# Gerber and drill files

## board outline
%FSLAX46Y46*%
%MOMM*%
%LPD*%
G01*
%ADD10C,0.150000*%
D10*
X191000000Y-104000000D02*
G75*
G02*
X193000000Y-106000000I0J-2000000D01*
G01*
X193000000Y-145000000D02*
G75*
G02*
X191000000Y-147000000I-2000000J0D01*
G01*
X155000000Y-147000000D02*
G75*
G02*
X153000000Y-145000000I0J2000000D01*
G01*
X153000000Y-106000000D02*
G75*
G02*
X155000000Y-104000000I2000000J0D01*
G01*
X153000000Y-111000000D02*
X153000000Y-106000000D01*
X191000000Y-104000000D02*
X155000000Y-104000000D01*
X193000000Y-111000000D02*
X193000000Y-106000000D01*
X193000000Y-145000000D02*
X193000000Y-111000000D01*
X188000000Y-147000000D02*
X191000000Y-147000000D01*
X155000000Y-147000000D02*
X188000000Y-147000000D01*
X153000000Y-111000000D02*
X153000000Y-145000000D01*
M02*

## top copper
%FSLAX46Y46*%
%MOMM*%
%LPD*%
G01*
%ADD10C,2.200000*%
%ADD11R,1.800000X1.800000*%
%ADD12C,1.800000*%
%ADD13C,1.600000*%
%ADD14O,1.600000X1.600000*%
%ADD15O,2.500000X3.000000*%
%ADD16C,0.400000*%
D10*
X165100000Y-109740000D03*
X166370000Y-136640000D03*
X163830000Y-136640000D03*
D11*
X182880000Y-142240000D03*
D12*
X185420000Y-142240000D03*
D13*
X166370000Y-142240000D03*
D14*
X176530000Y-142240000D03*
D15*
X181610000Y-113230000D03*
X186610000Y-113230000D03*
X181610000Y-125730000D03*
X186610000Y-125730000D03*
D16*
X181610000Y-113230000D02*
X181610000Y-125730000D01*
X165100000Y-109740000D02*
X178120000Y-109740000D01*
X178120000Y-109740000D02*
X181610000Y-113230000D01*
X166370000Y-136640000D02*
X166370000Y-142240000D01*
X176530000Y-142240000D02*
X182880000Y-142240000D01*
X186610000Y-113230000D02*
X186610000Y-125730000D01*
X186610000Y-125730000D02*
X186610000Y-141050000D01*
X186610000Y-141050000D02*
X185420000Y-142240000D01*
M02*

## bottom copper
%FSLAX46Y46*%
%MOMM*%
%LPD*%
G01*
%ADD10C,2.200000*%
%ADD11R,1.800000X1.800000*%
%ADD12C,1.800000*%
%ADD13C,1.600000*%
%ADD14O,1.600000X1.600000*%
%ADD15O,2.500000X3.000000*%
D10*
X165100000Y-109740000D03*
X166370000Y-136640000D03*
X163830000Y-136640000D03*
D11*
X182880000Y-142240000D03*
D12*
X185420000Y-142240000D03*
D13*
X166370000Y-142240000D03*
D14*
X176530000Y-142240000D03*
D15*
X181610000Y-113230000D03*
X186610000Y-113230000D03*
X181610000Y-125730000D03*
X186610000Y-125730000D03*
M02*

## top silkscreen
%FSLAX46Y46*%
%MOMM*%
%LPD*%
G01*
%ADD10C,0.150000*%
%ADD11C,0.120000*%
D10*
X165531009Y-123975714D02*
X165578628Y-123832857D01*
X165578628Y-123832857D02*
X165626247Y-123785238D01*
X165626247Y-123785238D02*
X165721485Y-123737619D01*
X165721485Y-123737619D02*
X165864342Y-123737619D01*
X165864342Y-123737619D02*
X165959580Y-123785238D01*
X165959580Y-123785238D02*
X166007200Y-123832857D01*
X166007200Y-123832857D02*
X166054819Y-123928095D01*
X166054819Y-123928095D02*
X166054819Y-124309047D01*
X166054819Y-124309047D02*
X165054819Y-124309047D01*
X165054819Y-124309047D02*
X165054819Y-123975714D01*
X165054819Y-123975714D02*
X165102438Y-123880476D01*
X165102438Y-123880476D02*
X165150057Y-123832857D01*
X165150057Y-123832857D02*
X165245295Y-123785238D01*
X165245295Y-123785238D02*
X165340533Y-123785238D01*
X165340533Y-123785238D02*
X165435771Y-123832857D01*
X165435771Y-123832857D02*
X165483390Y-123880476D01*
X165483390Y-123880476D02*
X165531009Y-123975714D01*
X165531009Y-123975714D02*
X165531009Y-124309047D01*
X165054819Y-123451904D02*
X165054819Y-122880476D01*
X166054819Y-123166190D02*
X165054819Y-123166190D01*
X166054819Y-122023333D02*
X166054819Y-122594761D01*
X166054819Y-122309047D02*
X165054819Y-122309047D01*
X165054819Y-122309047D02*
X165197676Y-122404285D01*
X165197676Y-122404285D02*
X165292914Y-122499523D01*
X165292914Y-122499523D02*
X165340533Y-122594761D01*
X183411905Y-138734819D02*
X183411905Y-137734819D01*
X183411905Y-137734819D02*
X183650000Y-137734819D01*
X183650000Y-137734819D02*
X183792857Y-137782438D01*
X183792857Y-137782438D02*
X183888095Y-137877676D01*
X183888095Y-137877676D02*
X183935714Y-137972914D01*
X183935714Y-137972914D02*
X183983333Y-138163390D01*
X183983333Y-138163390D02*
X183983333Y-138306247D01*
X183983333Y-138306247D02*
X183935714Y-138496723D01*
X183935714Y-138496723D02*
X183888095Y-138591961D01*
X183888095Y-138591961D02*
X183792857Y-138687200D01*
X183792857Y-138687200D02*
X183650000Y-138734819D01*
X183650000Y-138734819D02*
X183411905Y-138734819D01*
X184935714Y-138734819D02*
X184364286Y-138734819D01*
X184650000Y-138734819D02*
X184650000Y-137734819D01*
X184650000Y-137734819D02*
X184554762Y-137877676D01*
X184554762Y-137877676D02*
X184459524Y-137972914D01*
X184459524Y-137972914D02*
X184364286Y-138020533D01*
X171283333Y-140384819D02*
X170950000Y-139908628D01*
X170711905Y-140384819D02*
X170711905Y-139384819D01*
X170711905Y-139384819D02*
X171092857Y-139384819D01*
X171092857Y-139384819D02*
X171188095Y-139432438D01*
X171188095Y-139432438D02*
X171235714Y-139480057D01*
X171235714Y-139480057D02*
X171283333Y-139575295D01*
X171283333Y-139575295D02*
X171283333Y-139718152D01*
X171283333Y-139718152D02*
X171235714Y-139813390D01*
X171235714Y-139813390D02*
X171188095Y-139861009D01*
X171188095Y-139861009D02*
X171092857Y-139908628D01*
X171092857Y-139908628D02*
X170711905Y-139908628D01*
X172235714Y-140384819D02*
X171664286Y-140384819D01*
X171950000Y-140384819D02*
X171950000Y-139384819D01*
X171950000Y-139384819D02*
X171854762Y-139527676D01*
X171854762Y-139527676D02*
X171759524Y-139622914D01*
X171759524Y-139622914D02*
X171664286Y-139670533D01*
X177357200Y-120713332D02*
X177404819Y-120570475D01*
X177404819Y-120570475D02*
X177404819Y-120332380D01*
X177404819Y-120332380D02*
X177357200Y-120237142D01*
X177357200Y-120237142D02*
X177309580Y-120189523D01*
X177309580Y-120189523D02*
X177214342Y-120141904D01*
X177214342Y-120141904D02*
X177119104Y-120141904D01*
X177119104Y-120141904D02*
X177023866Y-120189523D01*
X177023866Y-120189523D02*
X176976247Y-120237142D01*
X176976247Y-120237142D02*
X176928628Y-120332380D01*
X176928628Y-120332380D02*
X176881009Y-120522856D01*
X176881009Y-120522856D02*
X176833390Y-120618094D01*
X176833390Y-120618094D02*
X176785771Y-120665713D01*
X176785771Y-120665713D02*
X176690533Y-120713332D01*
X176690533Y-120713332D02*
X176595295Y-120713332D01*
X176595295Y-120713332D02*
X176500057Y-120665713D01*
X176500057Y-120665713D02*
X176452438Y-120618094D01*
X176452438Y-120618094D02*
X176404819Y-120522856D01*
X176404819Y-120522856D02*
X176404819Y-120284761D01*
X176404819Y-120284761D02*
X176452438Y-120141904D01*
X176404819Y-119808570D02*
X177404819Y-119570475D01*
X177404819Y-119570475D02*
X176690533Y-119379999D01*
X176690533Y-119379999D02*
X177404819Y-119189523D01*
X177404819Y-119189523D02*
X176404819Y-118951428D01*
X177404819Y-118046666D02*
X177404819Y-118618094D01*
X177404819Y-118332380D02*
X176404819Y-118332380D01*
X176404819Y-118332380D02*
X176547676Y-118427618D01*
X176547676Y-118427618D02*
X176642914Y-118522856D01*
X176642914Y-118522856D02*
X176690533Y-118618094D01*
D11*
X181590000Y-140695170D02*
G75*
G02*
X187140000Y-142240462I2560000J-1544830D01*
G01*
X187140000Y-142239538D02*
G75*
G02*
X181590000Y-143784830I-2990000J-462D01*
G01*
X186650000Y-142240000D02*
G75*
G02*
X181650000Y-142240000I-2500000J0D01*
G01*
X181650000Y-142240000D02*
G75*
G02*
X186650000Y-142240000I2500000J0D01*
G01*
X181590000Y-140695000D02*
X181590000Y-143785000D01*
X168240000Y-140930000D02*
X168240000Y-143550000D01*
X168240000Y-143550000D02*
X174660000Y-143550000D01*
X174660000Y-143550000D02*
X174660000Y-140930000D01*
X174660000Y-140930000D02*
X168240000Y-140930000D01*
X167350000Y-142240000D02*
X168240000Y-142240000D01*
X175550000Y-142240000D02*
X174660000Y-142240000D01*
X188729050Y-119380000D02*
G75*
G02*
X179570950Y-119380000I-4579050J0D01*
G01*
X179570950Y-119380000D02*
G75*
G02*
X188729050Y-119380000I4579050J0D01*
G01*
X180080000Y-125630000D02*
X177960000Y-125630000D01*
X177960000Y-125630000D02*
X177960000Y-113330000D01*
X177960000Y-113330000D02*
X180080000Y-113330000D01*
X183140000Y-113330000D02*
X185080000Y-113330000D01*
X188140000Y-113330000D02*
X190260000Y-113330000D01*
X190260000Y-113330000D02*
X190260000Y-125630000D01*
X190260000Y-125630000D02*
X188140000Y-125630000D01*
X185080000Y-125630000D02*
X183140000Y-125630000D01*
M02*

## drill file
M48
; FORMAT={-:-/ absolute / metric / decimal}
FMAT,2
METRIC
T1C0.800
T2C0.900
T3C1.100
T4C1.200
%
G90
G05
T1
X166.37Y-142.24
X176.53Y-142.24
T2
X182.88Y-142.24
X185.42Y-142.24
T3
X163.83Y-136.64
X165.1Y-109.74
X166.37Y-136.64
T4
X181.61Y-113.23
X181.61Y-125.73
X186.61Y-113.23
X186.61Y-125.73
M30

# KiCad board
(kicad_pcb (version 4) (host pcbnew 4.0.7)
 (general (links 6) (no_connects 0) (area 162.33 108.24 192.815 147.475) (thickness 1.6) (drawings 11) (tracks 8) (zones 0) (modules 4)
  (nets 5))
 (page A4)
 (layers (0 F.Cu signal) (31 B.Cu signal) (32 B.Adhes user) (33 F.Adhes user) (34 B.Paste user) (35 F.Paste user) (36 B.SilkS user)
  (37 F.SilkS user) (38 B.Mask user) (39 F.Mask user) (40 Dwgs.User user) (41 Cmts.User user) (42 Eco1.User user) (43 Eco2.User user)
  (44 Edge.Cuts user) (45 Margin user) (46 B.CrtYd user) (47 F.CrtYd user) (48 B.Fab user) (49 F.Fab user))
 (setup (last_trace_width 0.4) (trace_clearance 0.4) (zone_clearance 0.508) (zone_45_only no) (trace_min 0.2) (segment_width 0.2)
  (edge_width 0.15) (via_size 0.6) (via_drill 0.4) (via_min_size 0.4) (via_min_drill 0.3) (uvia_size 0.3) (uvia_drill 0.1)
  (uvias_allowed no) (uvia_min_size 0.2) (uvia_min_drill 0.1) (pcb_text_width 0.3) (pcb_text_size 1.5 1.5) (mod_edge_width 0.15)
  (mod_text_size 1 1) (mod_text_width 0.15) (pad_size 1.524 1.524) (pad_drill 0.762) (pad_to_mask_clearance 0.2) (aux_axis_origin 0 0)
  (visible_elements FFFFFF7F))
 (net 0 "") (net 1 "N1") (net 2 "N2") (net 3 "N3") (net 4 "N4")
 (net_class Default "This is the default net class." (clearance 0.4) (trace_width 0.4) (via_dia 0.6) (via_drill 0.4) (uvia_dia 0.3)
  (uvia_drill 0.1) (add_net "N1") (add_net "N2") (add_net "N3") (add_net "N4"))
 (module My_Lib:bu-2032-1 (layer F.Cu) (at 165.1 123.19 90)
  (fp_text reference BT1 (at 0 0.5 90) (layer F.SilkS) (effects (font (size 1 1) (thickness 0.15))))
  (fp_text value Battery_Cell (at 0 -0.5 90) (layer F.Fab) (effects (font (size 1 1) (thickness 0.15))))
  (pad 1 thru_hole circle (at 13.45 0 90) (size 2.2 2.2) (drill 1.1) (layers *.Cu *.Mask) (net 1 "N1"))
  (pad 2 thru_hole circle (at -13.45 1.27 90) (size 2.2 2.2) (drill 1.1) (layers *.Cu *.Mask) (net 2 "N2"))
  (pad 3 thru_hole circle (at -13.45 -1.27 90) (size 2.2 2.2) (drill 1.1) (layers *.Cu *.Mask)))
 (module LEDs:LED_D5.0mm (layer F.Cu) (at 182.88 142.24)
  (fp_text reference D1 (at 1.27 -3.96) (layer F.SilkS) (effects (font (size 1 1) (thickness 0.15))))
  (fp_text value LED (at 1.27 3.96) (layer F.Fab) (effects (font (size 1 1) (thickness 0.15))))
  (fp_arc (start 1.27 0) (end -1.29 -1.54483) (angle 148.9) (layer F.SilkS) (width 0.12))
  (fp_arc (start 1.27 0) (end -1.29 1.54483) (angle -148.9) (layer F.SilkS) (width 0.12))
  (fp_circle (center 1.27 0) (end 3.77 0) (layer F.SilkS) (width 0.12))
  (fp_line (start -1.29 -1.545) (end -1.29 1.545) (layer F.SilkS) (width 0.12))
  (pad 1 thru_hole rect (at 0 0) (size 1.8 1.8) (drill 0.9) (layers *.Cu *.Mask) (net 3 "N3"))
  (pad 2 thru_hole circle (at 2.54 0) (size 1.8 1.8) (drill 0.9) (layers *.Cu *.Mask) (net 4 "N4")))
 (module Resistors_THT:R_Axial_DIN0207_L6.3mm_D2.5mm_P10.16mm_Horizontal (layer F.Cu) (at 166.37 142.24)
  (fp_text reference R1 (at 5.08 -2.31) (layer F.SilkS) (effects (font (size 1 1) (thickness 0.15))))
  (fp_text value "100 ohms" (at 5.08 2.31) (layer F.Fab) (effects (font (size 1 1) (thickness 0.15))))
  (fp_line (start 1.87 -1.31) (end 1.87 1.31) (layer F.SilkS) (width 0.12))
  (fp_line (start 1.87 1.31) (end 8.29 1.31) (layer F.SilkS) (width 0.12))
  (fp_line (start 8.29 1.31) (end 8.29 -1.31) (layer F.SilkS) (width 0.12))
  (fp_line (start 8.29 -1.31) (end 1.87 -1.31) (layer F.SilkS) (width 0.12))
  (fp_line (start 0.98 0) (end 1.87 0) (layer F.SilkS) (width 0.12))
  (fp_line (start 9.18 0) (end 8.29 0) (layer F.SilkS) (width 0.12))
  (pad 1 thru_hole circle (at 0 0) (size 1.6 1.6) (drill 0.8) (layers *.Cu *.Mask) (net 2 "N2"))
  (pad 2 thru_hole oval (at 10.16 0) (size 1.6 1.6) (drill 0.8) (layers *.Cu *.Mask) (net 3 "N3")))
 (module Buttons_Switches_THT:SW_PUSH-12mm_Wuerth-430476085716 (layer F.Cu) (at 181.61 125.73 90)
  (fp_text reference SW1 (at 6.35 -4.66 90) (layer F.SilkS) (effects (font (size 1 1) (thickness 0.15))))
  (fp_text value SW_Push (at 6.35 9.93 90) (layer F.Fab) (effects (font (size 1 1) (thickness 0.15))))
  (fp_circle (center 6.35 2.54) (end 10.92905 2.54) (layer F.SilkS) (width 0.12))
  (fp_line (start 0.1 -1.53) (end 0.1 -3.65) (layer F.SilkS) (width 0.12))
  (fp_line (start 0.1 -3.65) (end 12.4 -3.65) (layer F.SilkS) (width 0.12))
  (fp_line (start 12.4 -3.65) (end 12.4 -1.53) (layer F.SilkS) (width 0.12))
  (fp_line (start 12.4 1.53) (end 12.4 3.47) (layer F.SilkS) (width 0.12))
  (fp_line (start 12.4 6.53) (end 12.4 8.65) (layer F.SilkS) (width 0.12))
  (fp_line (start 12.4 8.65) (end 0.1 8.65) (layer F.SilkS) (width 0.12))
  (fp_line (start 0.1 8.65) (end 0.1 6.53) (layer F.SilkS) (width 0.12))
  (fp_line (start 0.1 3.47) (end 0.1 1.53) (layer F.SilkS) (width 0.12))
  (pad 1 thru_hole oval (at 12.5 0 90) (size 3 2.5) (drill 1.2) (layers *.Cu *.Mask) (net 1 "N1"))
  (pad 2 thru_hole oval (at 12.5 5 90) (size 3 2.5) (drill 1.2) (layers *.Cu *.Mask) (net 4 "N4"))
  (pad 1 thru_hole oval (at 0 0 90) (size 3 2.5) (drill 1.2) (layers *.Cu *.Mask) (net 1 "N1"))
  (pad 2 thru_hole oval (at 0 5 90) (size 3 2.5) (drill 1.2) (layers *.Cu *.Mask) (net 4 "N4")))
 (gr_arc (start 191 106) (end 191 104) (angle 90) (layer Edge.Cuts) (width 0.15))
 (gr_arc (start 191 145) (end 193 145) (angle 90) (layer Edge.Cuts) (width 0.15))
 (gr_arc (start 155 145) (end 155 147) (angle 90) (layer Edge.Cuts) (width 0.15))
 (gr_arc (start 155 106) (end 153 106) (angle 90) (layer Edge.Cuts) (width 0.15))
 (gr_line (start 153 111) (end 153 106) (angle 90) (layer Edge.Cuts) (width 0.15))
 (gr_line (start 191 104) (end 155 104) (angle 90) (layer Edge.Cuts) (width 0.15))
 (gr_line (start 193 111) (end 193 106) (angle 90) (layer Edge.Cuts) (width 0.15))
 (gr_line (start 193 145) (end 193 111) (angle 90) (layer Edge.Cuts) (width 0.15))
 (gr_line (start 188 147) (end 191 147) (angle 90) (layer Edge.Cuts) (width 0.15))
 (gr_line (start 155 147) (end 188 147) (angle 90) (layer Edge.Cuts) (width 0.15))
 (gr_line (start 153 111) (end 153 145) (angle 90) (layer Edge.Cuts) (width 0.15))
 (segment (start 181.61 113.23) (end 181.61 125.73) (width 0.4) (layer F.Cu) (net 1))
 (segment (start 165.1 109.74) (end 178.12 109.74) (width 0.4) (layer F.Cu) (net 1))
 (segment (start 178.12 109.74) (end 181.61 113.23) (width 0.4) (layer F.Cu) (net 1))
 (segment (start 166.37 136.64) (end 166.37 142.24) (width 0.4) (layer F.Cu) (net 2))
 (segment (start 176.53 142.24) (end 182.88 142.24) (width 0.4) (layer F.Cu) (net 3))
 (segment (start 186.61 113.23) (end 186.61 125.73) (width 0.4) (layer F.Cu) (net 4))
 (segment (start 186.61 125.73) (end 186.61 141.05) (width 0.4) (layer F.Cu) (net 4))
 (segment (start 186.61 141.05) (end 185.42 142.24) (width 0.4) (layer F.Cu) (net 4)))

